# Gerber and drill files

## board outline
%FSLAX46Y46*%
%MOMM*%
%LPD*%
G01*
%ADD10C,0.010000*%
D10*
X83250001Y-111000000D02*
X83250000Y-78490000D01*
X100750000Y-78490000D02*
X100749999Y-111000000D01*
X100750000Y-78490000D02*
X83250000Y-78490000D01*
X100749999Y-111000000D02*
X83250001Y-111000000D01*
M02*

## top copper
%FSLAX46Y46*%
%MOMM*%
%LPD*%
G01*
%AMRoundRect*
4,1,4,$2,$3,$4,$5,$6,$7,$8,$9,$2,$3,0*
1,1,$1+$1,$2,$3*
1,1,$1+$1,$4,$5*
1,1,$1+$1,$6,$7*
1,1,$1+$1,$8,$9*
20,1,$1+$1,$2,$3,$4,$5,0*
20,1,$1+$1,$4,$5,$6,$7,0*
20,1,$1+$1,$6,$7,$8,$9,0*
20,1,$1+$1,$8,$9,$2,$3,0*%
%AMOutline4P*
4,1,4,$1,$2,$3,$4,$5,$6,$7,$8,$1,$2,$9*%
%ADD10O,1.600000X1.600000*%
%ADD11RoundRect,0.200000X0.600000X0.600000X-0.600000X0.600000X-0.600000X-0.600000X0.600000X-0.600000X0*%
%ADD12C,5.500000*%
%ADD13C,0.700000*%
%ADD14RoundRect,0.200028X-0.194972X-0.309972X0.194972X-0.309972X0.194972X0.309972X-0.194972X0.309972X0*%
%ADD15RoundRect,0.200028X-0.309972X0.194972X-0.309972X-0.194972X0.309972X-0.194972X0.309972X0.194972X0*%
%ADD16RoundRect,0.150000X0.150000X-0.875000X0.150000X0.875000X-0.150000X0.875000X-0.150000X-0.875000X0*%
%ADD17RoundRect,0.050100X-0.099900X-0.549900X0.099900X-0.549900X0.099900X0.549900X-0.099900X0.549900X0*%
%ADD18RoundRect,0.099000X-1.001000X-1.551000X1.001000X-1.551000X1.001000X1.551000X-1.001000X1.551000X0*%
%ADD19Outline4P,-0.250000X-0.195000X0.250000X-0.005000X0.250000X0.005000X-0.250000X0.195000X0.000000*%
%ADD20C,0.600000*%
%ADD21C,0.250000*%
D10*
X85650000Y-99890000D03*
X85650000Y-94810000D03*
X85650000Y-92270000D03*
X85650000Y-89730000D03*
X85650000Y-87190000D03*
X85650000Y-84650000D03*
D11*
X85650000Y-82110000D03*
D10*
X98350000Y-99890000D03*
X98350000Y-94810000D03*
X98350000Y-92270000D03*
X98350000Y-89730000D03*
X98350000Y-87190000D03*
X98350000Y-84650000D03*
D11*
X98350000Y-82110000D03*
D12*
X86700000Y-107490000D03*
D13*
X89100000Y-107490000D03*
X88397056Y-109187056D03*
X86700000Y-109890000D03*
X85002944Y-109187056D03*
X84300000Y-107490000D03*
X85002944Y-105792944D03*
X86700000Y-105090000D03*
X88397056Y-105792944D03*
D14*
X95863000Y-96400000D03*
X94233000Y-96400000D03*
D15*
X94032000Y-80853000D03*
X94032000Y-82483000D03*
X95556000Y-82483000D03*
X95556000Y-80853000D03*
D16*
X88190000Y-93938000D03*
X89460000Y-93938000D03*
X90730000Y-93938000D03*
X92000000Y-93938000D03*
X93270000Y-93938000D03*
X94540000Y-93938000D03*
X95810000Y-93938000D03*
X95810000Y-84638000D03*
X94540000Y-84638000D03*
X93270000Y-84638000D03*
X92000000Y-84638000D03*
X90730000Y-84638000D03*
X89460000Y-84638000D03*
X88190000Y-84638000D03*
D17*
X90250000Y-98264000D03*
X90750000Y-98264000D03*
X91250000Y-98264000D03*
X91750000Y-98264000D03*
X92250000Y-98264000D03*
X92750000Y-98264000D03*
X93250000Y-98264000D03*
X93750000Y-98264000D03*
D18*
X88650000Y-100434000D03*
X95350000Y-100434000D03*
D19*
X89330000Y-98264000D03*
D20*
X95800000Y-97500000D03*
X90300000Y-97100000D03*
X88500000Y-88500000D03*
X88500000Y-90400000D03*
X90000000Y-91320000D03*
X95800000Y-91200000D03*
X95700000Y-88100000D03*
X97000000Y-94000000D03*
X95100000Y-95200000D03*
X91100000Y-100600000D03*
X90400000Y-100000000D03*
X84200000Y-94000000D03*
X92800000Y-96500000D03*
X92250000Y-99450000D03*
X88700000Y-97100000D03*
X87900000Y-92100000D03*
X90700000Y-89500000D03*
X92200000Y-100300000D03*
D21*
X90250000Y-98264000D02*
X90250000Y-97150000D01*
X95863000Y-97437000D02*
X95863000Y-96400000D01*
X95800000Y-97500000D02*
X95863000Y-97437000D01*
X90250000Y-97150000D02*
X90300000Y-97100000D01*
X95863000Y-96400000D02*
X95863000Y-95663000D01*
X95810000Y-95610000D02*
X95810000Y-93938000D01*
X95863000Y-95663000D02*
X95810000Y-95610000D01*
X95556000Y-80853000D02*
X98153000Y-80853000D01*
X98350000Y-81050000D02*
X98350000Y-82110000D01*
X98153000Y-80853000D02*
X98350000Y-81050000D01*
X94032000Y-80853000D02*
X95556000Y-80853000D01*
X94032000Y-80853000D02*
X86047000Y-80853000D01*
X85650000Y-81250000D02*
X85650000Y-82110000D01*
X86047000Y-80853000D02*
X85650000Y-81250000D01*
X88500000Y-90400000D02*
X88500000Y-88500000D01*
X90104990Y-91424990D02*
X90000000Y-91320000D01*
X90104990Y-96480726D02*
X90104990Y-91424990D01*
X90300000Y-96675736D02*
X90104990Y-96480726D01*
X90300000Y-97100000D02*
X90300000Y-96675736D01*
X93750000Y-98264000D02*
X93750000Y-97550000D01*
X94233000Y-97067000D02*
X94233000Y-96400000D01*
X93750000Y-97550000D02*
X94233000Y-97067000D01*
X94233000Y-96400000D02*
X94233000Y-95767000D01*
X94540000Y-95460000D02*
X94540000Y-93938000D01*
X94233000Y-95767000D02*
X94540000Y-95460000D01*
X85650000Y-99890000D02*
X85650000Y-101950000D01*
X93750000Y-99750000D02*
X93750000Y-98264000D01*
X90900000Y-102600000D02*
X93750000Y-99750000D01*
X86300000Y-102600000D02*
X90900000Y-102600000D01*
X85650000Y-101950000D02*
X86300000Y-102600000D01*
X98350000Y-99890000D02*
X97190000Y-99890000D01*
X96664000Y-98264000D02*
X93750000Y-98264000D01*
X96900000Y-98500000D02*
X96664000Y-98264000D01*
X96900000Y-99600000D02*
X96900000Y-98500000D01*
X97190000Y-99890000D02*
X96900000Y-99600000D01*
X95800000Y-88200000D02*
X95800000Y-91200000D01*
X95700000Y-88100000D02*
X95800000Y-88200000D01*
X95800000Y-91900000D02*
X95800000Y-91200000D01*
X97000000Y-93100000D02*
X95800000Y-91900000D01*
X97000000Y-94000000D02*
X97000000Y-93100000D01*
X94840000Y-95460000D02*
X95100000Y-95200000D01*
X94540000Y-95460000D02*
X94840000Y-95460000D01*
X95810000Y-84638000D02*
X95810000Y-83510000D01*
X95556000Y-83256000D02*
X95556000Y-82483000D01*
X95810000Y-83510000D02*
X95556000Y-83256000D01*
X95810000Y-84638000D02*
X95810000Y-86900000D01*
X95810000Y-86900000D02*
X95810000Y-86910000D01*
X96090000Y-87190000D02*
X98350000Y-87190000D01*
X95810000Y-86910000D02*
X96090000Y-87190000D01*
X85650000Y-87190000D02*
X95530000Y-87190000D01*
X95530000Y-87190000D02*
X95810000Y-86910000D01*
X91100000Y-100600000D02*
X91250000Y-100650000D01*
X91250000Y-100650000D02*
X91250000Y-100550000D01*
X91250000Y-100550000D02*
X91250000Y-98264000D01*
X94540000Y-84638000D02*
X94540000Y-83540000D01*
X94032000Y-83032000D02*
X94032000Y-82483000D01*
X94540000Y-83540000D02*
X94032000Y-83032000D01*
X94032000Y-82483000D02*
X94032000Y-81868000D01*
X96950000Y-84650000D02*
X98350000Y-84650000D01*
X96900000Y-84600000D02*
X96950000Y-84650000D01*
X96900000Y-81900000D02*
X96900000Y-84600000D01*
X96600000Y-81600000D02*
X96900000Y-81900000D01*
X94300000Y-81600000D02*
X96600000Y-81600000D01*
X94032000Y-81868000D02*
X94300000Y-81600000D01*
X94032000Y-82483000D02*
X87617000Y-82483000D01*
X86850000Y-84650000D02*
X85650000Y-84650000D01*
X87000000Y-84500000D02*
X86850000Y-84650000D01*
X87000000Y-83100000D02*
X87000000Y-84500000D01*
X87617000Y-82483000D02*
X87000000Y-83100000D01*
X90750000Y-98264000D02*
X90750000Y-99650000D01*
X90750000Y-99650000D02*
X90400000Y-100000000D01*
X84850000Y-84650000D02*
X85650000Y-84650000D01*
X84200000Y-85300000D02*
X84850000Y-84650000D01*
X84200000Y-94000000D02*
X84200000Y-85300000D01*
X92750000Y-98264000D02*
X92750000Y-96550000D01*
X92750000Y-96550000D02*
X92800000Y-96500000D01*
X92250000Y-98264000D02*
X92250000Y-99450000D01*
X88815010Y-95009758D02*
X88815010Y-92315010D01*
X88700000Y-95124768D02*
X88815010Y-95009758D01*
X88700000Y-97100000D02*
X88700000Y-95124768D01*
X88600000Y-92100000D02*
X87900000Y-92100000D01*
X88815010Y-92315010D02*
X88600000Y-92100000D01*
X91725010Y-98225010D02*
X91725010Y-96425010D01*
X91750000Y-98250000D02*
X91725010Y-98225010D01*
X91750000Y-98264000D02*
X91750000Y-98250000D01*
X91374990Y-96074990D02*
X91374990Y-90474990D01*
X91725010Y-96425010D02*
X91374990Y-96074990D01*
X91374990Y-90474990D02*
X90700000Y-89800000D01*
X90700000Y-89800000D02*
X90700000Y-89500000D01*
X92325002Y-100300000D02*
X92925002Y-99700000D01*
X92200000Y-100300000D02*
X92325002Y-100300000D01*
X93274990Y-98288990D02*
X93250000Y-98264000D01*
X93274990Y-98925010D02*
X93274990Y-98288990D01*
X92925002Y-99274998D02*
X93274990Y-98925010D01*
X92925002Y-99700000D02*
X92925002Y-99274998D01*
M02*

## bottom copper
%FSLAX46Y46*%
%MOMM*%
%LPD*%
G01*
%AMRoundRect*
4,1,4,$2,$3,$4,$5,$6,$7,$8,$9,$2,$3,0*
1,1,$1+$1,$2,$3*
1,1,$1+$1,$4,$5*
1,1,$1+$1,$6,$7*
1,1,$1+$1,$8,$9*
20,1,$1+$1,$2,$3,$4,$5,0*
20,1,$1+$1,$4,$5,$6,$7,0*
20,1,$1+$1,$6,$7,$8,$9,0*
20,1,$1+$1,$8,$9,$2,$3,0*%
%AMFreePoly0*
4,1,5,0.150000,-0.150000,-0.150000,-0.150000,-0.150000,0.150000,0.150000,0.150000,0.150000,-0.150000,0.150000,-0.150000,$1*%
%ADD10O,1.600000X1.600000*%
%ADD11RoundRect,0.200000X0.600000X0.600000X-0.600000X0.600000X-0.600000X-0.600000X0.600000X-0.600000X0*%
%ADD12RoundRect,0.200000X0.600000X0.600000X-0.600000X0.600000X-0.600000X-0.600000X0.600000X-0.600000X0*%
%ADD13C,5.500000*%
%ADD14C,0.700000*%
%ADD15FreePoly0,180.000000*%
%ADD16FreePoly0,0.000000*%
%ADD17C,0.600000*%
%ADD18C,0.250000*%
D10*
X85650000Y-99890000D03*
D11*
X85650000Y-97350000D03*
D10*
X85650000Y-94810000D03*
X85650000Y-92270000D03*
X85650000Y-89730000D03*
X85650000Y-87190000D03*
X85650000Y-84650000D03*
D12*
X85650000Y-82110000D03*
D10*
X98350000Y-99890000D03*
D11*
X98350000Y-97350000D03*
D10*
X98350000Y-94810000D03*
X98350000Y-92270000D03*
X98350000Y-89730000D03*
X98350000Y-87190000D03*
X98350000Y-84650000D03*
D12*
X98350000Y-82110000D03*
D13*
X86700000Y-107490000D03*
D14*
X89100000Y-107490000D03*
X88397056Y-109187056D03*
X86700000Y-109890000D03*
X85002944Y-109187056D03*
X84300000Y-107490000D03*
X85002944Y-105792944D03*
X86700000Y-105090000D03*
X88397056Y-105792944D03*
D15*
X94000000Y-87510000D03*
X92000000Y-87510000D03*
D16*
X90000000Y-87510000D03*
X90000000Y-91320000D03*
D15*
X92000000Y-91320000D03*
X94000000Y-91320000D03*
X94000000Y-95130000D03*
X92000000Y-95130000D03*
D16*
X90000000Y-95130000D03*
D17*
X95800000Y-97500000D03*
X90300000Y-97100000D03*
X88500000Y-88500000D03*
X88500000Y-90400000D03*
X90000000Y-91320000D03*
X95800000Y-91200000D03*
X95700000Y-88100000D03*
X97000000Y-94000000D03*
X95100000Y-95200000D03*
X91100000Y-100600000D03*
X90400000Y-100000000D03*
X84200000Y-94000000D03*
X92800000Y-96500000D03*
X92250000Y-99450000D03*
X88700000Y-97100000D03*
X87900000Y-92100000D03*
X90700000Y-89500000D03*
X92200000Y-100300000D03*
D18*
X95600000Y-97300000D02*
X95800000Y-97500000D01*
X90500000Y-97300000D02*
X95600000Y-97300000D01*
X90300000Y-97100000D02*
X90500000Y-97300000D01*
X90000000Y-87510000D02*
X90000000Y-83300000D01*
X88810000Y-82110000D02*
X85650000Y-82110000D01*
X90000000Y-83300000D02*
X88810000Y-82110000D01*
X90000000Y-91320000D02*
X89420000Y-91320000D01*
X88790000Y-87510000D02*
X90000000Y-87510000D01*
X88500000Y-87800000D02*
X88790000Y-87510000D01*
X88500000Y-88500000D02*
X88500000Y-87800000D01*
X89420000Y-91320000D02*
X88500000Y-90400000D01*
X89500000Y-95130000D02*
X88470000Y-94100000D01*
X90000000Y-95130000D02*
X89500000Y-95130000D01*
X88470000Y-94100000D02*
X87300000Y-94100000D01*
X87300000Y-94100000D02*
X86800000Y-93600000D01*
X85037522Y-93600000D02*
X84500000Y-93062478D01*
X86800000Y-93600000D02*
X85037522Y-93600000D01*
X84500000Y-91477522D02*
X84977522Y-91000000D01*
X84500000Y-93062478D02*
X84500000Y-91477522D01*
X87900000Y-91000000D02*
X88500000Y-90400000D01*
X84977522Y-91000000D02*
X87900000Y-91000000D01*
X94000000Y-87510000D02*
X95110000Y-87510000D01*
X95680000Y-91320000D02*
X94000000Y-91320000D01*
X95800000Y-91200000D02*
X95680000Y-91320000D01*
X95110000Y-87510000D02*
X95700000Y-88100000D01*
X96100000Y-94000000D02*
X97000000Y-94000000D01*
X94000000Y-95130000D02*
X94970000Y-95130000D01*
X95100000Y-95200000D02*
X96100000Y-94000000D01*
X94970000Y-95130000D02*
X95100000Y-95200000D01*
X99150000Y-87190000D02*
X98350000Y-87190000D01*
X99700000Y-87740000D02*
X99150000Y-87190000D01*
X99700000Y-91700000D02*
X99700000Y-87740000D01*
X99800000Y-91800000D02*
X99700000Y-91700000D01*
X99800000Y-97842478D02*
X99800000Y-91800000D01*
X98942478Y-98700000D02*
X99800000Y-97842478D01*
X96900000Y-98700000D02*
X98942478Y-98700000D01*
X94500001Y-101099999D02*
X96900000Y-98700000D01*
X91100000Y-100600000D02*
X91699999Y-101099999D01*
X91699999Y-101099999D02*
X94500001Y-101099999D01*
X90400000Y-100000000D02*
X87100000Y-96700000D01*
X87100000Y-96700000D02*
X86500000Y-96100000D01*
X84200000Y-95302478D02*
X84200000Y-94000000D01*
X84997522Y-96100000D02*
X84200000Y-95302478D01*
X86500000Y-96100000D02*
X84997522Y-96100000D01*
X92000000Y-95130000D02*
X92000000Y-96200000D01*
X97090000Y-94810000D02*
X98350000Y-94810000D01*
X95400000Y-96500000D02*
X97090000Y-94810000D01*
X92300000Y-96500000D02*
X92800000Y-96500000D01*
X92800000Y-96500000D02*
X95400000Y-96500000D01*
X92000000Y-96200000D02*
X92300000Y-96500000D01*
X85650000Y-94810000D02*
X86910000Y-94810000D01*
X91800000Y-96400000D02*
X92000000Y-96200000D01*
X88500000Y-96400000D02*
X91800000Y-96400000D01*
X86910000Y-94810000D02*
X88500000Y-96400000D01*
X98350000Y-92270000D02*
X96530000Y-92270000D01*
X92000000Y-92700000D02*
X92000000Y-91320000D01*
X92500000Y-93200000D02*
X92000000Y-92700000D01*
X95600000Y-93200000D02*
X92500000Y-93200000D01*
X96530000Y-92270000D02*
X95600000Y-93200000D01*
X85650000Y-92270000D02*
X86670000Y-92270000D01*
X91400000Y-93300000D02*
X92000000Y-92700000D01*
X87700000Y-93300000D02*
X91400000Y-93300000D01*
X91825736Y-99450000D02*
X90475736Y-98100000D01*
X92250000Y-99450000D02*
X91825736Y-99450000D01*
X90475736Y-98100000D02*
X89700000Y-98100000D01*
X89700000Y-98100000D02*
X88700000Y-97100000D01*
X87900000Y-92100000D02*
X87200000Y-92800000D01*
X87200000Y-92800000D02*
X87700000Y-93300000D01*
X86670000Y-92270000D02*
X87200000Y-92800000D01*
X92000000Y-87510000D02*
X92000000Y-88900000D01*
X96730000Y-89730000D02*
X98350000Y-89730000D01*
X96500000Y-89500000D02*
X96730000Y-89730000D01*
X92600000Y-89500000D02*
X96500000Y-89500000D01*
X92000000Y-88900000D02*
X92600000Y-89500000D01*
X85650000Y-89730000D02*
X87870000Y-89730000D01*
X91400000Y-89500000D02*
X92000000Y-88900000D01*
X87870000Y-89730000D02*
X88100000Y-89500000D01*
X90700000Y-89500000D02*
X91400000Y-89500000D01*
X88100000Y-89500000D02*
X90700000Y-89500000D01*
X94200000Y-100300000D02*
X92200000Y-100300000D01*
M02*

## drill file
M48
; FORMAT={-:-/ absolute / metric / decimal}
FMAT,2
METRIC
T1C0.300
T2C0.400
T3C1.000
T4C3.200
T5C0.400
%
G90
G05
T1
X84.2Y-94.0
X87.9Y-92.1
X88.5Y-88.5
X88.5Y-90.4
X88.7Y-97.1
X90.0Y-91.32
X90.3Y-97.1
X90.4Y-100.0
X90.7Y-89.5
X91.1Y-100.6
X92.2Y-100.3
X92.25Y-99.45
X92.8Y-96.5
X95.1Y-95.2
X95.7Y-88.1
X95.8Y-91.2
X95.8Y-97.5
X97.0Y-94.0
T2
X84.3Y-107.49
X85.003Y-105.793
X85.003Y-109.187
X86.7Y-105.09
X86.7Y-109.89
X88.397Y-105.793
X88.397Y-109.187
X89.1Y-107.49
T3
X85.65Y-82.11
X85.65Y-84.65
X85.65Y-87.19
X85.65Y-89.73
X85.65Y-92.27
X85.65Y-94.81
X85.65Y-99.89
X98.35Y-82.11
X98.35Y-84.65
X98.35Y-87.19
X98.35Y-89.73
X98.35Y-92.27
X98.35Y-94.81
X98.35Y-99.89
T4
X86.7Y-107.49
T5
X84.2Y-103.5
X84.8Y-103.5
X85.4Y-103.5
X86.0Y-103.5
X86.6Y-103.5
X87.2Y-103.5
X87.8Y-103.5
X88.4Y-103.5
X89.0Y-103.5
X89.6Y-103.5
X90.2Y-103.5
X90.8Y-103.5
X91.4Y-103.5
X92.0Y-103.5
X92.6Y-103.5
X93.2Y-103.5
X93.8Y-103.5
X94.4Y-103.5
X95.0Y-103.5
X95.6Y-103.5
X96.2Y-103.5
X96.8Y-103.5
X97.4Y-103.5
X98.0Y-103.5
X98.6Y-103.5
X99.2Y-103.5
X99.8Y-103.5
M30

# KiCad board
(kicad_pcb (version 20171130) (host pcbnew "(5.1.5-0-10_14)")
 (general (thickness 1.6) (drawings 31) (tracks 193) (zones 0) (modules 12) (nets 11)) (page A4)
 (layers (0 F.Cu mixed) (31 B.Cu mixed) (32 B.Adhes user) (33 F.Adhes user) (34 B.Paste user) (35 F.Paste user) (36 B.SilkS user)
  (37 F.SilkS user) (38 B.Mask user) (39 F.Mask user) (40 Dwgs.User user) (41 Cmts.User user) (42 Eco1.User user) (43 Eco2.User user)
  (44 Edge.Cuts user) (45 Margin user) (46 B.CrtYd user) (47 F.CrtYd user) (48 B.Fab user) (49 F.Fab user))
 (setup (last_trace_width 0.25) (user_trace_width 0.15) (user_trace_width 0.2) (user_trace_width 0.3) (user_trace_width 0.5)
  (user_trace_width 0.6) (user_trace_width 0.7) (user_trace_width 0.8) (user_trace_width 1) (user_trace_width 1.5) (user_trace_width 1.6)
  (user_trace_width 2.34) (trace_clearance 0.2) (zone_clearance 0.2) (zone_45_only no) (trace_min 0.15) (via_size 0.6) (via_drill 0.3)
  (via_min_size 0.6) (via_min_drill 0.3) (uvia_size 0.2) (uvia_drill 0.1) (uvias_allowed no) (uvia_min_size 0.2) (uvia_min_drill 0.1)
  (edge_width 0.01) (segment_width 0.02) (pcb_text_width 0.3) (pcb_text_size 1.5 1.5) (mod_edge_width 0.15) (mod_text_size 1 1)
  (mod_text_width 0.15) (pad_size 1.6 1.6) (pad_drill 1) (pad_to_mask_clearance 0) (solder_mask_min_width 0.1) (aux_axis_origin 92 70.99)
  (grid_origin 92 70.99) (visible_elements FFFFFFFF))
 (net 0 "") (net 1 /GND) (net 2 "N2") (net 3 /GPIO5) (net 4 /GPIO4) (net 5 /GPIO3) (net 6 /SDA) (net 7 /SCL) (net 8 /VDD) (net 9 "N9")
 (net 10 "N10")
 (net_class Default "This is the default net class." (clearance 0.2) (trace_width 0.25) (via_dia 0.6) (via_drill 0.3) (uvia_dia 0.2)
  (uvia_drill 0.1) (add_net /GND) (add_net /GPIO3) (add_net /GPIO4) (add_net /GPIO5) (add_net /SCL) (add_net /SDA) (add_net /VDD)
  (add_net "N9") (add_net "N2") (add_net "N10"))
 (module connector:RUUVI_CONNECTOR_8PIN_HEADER (layer B.Cu) (at 85.65 82.11 180)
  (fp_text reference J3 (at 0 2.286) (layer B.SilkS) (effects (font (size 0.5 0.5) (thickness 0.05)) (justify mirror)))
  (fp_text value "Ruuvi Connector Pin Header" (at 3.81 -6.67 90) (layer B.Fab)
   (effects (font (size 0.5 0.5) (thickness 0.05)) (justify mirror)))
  (pad 8 thru_hole oval (at 0 -17.78 180) (size 1.6 1.6) (drill 1) (layers *.Cu *.Mask) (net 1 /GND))
  (pad 7 smd roundrect (at 0 -15.24 180) (size 1.6 1.6) (layers B.Cu B.Paste B.Mask) (roundrect_rratio 0.125) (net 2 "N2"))
  (pad 6 thru_hole oval (at 0 -12.7 180) (size 1.6 1.6) (drill 1) (layers *.Cu *.Mask) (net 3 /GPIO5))
  (pad 5 thru_hole oval (at 0 -10.16 180) (size 1.6 1.6) (drill 1) (layers *.Cu *.Mask) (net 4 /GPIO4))
  (pad 4 thru_hole oval (at 0 -7.62 180) (size 1.6 1.6) (drill 1) (layers *.Cu *.Mask) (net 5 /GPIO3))
  (pad 3 thru_hole oval (at 0 -5.08 180) (size 1.6 1.6) (drill 1) (layers *.Cu *.Mask) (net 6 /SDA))
  (pad 2 thru_hole oval (at 0 -2.54 180) (size 1.6 1.6) (drill 1) (layers *.Cu *.Mask) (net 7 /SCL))
  (pad 1 thru_hole roundrect (at 0 0 180) (size 1.6 1.6) (drill 1) (layers *.Cu *.Mask) (roundrect_rratio 0.125) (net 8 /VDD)))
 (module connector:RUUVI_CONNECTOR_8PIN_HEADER (layer B.Cu) (at 98.35 82.11 180)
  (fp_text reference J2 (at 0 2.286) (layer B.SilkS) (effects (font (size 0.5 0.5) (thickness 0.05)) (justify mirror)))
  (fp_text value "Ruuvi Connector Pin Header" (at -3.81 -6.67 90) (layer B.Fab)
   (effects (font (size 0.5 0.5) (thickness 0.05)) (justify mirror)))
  (pad 8 thru_hole oval (at 0 -17.78 180) (size 1.6 1.6) (drill 1) (layers *.Cu *.Mask) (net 1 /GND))
  (pad 7 smd roundrect (at 0 -15.24 180) (size 1.6 1.6) (layers B.Cu B.Paste B.Mask) (roundrect_rratio 0.125) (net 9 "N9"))
  (pad 6 thru_hole oval (at 0 -12.7 180) (size 1.6 1.6) (drill 1) (layers *.Cu *.Mask) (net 3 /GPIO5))
  (pad 5 thru_hole oval (at 0 -10.16 180) (size 1.6 1.6) (drill 1) (layers *.Cu *.Mask) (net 4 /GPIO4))
  (pad 4 thru_hole oval (at 0 -7.62 180) (size 1.6 1.6) (drill 1) (layers *.Cu *.Mask) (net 5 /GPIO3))
  (pad 3 thru_hole oval (at 0 -5.08 180) (size 1.6 1.6) (drill 1) (layers *.Cu *.Mask) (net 6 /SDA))
  (pad 2 thru_hole oval (at 0 -2.54 180) (size 1.6 1.6) (drill 1) (layers *.Cu *.Mask) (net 7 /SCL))
  (pad 1 thru_hole roundrect (at 0 0 180) (size 1.6 1.6) (drill 1) (layers *.Cu *.Mask) (roundrect_rratio 0.125) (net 8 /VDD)))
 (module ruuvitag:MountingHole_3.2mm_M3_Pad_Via (layer F.Cu) (at 86.7 107.49)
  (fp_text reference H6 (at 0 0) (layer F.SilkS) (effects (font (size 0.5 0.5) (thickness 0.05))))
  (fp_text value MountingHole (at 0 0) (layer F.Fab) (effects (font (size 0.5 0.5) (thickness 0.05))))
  (pad 1 thru_hole circle (at 0 0) (size 5.5 5.5) (drill 3.2) (layers *.Cu *.Mask))
  (pad 1 thru_hole circle (at 2.4 0) (size 0.7 0.7) (drill 0.4) (layers *.Cu *.Mask))
  (pad 1 thru_hole circle (at 1.697056 1.697056) (size 0.7 0.7) (drill 0.4) (layers *.Cu *.Mask))
  (pad 1 thru_hole circle (at 0 2.4) (size 0.7 0.7) (drill 0.4) (layers *.Cu *.Mask))
  (pad 1 thru_hole circle (at -1.697056 1.697056) (size 0.7 0.7) (drill 0.4) (layers *.Cu *.Mask))
  (pad 1 thru_hole circle (at -2.4 0) (size 0.7 0.7) (drill 0.4) (layers *.Cu *.Mask))
  (pad 1 thru_hole circle (at -1.697056 -1.697056) (size 0.7 0.7) (drill 0.4) (layers *.Cu *.Mask))
  (pad 1 thru_hole circle (at 0 -2.4) (size 0.7 0.7) (drill 0.4) (layers *.Cu *.Mask))
  (pad 1 thru_hole circle (at 1.697056 -1.697056) (size 0.7 0.7) (drill 0.4) (layers *.Cu *.Mask)))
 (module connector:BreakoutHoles (layer F.Cu) (at 92 103.5)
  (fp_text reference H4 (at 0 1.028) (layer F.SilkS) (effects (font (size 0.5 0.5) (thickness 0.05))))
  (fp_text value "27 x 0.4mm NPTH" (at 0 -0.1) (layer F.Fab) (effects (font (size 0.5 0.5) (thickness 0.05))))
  (pad "" np_thru_hole circle (at -6.6 0) (size 0.4 0.4) (drill 0.4) (layers *.Cu *.Mask))
  (pad "" np_thru_hole circle (at -0.6 0) (size 0.4 0.4) (drill 0.4) (layers *.Cu *.Mask))
  (pad "" np_thru_hole circle (at -3.6 0) (size 0.4 0.4) (drill 0.4) (layers *.Cu *.Mask))
  (pad "" np_thru_hole circle (at -1.2 0) (size 0.4 0.4) (drill 0.4) (layers *.Cu *.Mask))
  (pad "" np_thru_hole circle (at -3 0) (size 0.4 0.4) (drill 0.4) (layers *.Cu *.Mask))
  (pad "" np_thru_hole circle (at -1.8 0) (size 0.4 0.4) (drill 0.4) (layers *.Cu *.Mask))
  (pad "" np_thru_hole circle (at -4.8 0) (size 0.4 0.4) (drill 0.4) (layers *.Cu *.Mask))
  (pad "" np_thru_hole circle (at -5.4 0) (size 0.4 0.4) (drill 0.4) (layers *.Cu *.Mask))
  (pad "" np_thru_hole circle (at -7.8 0) (size 0.4 0.4) (drill 0.4) (layers *.Cu *.Mask))
  (pad "" np_thru_hole circle (at -2.4 0) (size 0.4 0.4) (drill 0.4) (layers *.Cu *.Mask))
  (pad "" np_thru_hole circle (at -4.2 0) (size 0.4 0.4) (drill 0.4) (layers *.Cu *.Mask))
  (pad "" np_thru_hole circle (at -7.2 0) (size 0.4 0.4) (drill 0.4) (layers *.Cu *.Mask))
  (pad "" np_thru_hole circle (at -6 0) (size 0.4 0.4) (drill 0.4) (layers *.Cu *.Mask))
  (pad "" np_thru_hole circle (at 7.8 0) (size 0.4 0.4) (drill 0.4) (layers *.Cu *.Mask))
  (pad "" np_thru_hole circle (at 7.2 0) (size 0.4 0.4) (drill 0.4) (layers *.Cu *.Mask))
  (pad "" np_thru_hole circle (at 6.6 0) (size 0.4 0.4) (drill 0.4) (layers *.Cu *.Mask))
  (pad "" np_thru_hole circle (at 6 0) (size 0.4 0.4) (drill 0.4) (layers *.Cu *.Mask))
  (pad "" np_thru_hole circle (at 5.4 0) (size 0.4 0.4) (drill 0.4) (layers *.Cu *.Mask))
  (pad "" np_thru_hole circle (at 4.8 0) (size 0.4 0.4) (drill 0.4) (layers *.Cu *.Mask))
  (pad "" np_thru_hole circle (at 4.2 0) (size 0.4 0.4) (drill 0.4) (layers *.Cu *.Mask))
  (pad "" np_thru_hole circle (at 3.6 0) (size 0.4 0.4) (drill 0.4) (layers *.Cu *.Mask))
  (pad "" np_thru_hole circle (at 3 0) (size 0.4 0.4) (drill 0.4) (layers *.Cu *.Mask))
  (pad "" np_thru_hole circle (at 2.4 0) (size 0.4 0.4) (drill 0.4) (layers *.Cu *.Mask))
  (pad "" np_thru_hole circle (at 1.8 0) (size 0.4 0.4) (drill 0.4) (layers *.Cu *.Mask))
  (pad "" np_thru_hole circle (at 1.2 0) (size 0.4 0.4) (drill 0.4) (layers *.Cu *.Mask))
  (pad "" np_thru_hole circle (at 0.6 0) (size 0.4 0.4) (drill 0.4) (layers *.Cu *.Mask))
  (pad "" np_thru_hole circle (at 0 0) (size 0.4 0.4) (drill 0.4) (layers *.Cu *.Mask)))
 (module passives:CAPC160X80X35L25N (layer F.Cu) (at 95.048 96.4)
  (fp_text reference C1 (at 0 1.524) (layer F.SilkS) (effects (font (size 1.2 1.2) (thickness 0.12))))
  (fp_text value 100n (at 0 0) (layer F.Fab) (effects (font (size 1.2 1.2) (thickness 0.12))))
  (pad 2 smd roundrect (at 0.815 0) (size 0.79 1.02) (layers F.Cu F.Paste F.Mask) (roundrect_rratio 0.2532) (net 8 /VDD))
  (pad 1 smd roundrect (at -0.815 0) (size 0.79 1.02) (layers F.Cu F.Paste F.Mask) (roundrect_rratio 0.2532) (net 1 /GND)))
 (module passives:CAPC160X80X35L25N (layer F.Cu) (at 94.032 81.668 270)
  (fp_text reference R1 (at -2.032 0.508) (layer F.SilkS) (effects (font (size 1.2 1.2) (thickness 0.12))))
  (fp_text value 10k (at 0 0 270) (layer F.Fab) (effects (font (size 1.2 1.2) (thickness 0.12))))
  (pad 1 smd roundrect (at -0.815 0 270) (size 0.79 1.02) (layers F.Cu F.Paste F.Mask) (roundrect_rratio 0.2532) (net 8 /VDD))
  (pad 2 smd roundrect (at 0.815 0 270) (size 0.79 1.02) (layers F.Cu F.Paste F.Mask) (roundrect_rratio 0.2532) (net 7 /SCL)))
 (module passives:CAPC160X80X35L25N (layer F.Cu) (at 95.556 81.668 270)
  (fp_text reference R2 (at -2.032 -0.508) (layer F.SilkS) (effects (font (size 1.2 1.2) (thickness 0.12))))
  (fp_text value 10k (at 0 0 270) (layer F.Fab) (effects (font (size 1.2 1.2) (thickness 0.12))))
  (pad 2 smd roundrect (at 0.815 0 270) (size 0.79 1.02) (layers F.Cu F.Paste F.Mask) (roundrect_rratio 0.2532) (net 6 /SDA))
  (pad 1 smd roundrect (at -0.815 0 270) (size 0.79 1.02) (layers F.Cu F.Paste F.Mask) (roundrect_rratio 0.2532) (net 8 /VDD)))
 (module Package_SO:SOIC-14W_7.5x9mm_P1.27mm (layer F.Cu) (at 92 89.288 90)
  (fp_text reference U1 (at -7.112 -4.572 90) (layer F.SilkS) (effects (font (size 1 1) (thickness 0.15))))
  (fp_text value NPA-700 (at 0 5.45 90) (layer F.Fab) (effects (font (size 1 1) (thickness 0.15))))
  (pad 1 smd roundrect (at -4.65 -3.81 90) (size 2.05 0.6) (layers F.Cu F.Paste F.Mask) (roundrect_rratio 0.25))
  (pad 2 smd roundrect (at -4.65 -2.54 90) (size 2.05 0.6) (layers F.Cu F.Paste F.Mask) (roundrect_rratio 0.25))
  (pad 3 smd roundrect (at -4.65 -1.27 90) (size 2.05 0.6) (layers F.Cu F.Paste F.Mask) (roundrect_rratio 0.25))
  (pad 4 smd roundrect (at -4.65 0 90) (size 2.05 0.6) (layers F.Cu F.Paste F.Mask) (roundrect_rratio 0.25))
  (pad 5 smd roundrect (at -4.65 1.27 90) (size 2.05 0.6) (layers F.Cu F.Paste F.Mask) (roundrect_rratio 0.25))
  (pad 6 smd roundrect (at -4.65 2.54 90) (size 2.05 0.6) (layers F.Cu F.Paste F.Mask) (roundrect_rratio 0.25) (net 1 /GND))
  (pad 7 smd roundrect (at -4.65 3.81 90) (size 2.05 0.6) (layers F.Cu F.Paste F.Mask) (roundrect_rratio 0.25) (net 8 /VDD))
  (pad 8 smd roundrect (at 4.65 3.81 90) (size 2.05 0.6) (layers F.Cu F.Paste F.Mask) (roundrect_rratio 0.25) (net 6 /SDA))
  (pad 9 smd roundrect (at 4.65 2.54 90) (size 2.05 0.6) (layers F.Cu F.Paste F.Mask) (roundrect_rratio 0.25) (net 7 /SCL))
  (pad 10 smd roundrect (at 4.65 1.27 90) (size 2.05 0.6) (layers F.Cu F.Paste F.Mask) (roundrect_rratio 0.25))
  (pad 11 smd roundrect (at 4.65 0 90) (size 2.05 0.6) (layers F.Cu F.Paste F.Mask) (roundrect_rratio 0.25))
  (pad 12 smd roundrect (at 4.65 -1.27 90) (size 2.05 0.6) (layers F.Cu F.Paste F.Mask) (roundrect_rratio 0.25))
  (pad 13 smd roundrect (at 4.65 -2.54 90) (size 2.05 0.6) (layers F.Cu F.Paste F.Mask) (roundrect_rratio 0.25))
  (pad 14 smd roundrect (at 4.65 -3.81 90) (size 2.05 0.6) (layers F.Cu F.Paste F.Mask) (roundrect_rratio 0.25)))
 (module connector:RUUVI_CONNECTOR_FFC (layer F.Cu) (at 92 100.464)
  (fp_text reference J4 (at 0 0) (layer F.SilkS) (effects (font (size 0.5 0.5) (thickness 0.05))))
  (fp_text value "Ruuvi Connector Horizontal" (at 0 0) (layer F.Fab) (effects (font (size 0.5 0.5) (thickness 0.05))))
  (pad 1 smd roundrect (at -1.75 -2.2) (size 0.3 1.2) (layers F.Cu F.Paste F.Mask) (roundrect_rratio 0.167) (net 8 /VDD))
  (pad 2 smd roundrect (at -1.25 -2.2) (size 0.3 1.2) (layers F.Cu F.Paste F.Mask) (roundrect_rratio 0.167) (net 7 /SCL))
  (pad 3 smd roundrect (at -0.75 -2.2) (size 0.3 1.2) (layers F.Cu F.Paste F.Mask) (roundrect_rratio 0.167) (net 6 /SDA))
  (pad 4 smd roundrect (at -0.25 -2.2) (size 0.3 1.2) (layers F.Cu F.Paste F.Mask) (roundrect_rratio 0.167) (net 5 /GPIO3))
  (pad 5 smd roundrect (at 0.25 -2.2) (size 0.3 1.2) (layers F.Cu F.Paste F.Mask) (roundrect_rratio 0.167) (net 4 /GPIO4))
  (pad 6 smd roundrect (at 0.75 -2.2) (size 0.3 1.2) (layers F.Cu F.Paste F.Mask) (roundrect_rratio 0.167) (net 3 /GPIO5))
  (pad 7 smd roundrect (at 1.25 -2.2) (size 0.3 1.2) (layers F.Cu F.Paste F.Mask) (roundrect_rratio 0.167) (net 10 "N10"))
  (pad 8 smd roundrect (at 1.75 -2.2) (size 0.3 1.2) (layers F.Cu F.Paste F.Mask) (roundrect_rratio 0.167) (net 1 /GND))
  (pad ~ smd roundrect (at -3.35 -0.03) (size 2.2 3.3) (layers F.Cu F.Paste F.Mask) (roundrect_rratio 0.045))
  (pad ~ smd roundrect (at 3.35 -0.03) (size 2.2 3.3) (layers F.Cu F.Paste F.Mask) (roundrect_rratio 0.045))
  (pad ~ smd trapezoid (at -2.67 -2.2) (size 0.5 0.2) (rect_delta 0.19 0) (layers F.Cu F.Mask)))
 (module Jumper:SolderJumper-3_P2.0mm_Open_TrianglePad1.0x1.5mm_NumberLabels (layer B.Cu) (at 92 87.51 180)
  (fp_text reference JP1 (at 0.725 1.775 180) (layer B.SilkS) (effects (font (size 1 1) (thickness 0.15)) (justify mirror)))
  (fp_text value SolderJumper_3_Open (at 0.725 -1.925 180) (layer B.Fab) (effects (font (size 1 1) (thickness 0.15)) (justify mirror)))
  (pad "" smd rect (at 1.2 0 180) (size 1.5 1.5) (layers B.Mask))
  (pad "" smd rect (at -1.2 0 180) (size 1.5 1.5) (layers B.Mask))
  (pad 1 smd custom (at -2 0 180) (size 0.3 0.3) (layers B.Cu B.Mask) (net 1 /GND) (zone_connect 2)
   (options (clearance outline) (anchor rect)) (primitives))
  (pad 2 smd custom (at 0 0 180) (size 0.3 0.3) (layers B.Cu) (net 5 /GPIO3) (zone_connect 2) (options (clearance outline) (anchor rect))
   (primitives))
  (pad 3 smd custom (at 2 0) (size 0.3 0.3) (layers B.Cu B.Mask) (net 8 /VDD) (zone_connect 2) (options (clearance outline) (anchor rect))
   (primitives)))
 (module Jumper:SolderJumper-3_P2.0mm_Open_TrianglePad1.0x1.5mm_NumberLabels (layer B.Cu) (at 92 91.32 180)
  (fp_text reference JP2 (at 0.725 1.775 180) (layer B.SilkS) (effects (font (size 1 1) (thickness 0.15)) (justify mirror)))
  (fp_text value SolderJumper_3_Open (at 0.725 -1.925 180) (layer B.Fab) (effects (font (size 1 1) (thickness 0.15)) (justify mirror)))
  (pad 3 smd custom (at 2 0) (size 0.3 0.3) (layers B.Cu B.Mask) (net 8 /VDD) (zone_connect 2) (options (clearance outline) (anchor rect))
   (primitives))
  (pad 2 smd custom (at 0 0 180) (size 0.3 0.3) (layers B.Cu) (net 4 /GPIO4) (zone_connect 2) (options (clearance outline) (anchor rect))
   (primitives))
  (pad 1 smd custom (at -2 0 180) (size 0.3 0.3) (layers B.Cu B.Mask) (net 1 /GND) (zone_connect 2)
   (options (clearance outline) (anchor rect)) (primitives))
  (pad "" smd rect (at -1.2 0 180) (size 1.5 1.5) (layers B.Mask))
  (pad "" smd rect (at 1.2 0 180) (size 1.5 1.5) (layers B.Mask)))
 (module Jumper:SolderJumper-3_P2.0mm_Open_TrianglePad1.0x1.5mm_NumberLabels (layer B.Cu) (at 92 95.13 180)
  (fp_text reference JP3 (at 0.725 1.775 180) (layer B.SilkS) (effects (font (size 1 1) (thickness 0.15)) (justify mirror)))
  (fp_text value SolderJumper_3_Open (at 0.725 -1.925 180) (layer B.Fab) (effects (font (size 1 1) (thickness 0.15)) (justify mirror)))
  (pad "" smd rect (at 1.2 0 180) (size 1.5 1.5) (layers B.Mask))
  (pad "" smd rect (at -1.2 0 180) (size 1.5 1.5) (layers B.Mask))
  (pad 1 smd custom (at -2 0 180) (size 0.3 0.3) (layers B.Cu B.Mask) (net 1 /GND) (zone_connect 2)
   (options (clearance outline) (anchor rect)) (primitives))
  (pad 2 smd custom (at 0 0 180) (size 0.3 0.3) (layers B.Cu) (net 3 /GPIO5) (zone_connect 2) (options (clearance outline) (anchor rect))
   (primitives))
  (pad 3 smd custom (at 2 0) (size 0.3 0.3) (layers B.Cu B.Mask) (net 8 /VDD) (zone_connect 2) (options (clearance outline) (anchor rect))
   (primitives)))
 (gr_line (start 83.250001 111) (end 83.25 78.49) (layer Edge.Cuts) (width 0.01))
 (gr_line (start 100.75 78.49) (end 100.749999 111) (layer Edge.Cuts) (width 0.01))
 (gr_line (start 100.75 78.49) (end 83.25 78.49) (layer Edge.Cuts) (width 0.01))
 (gr_line (start 100.749999 111) (end 83.250001 111) (layer Edge.Cuts) (width 0.01))
 (segment (start 90.25 98.264) (end 90.25 97.15) (width 0.25) (layer F.Cu) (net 8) (status 400000))
 (segment (start 95.863 97.437) (end 95.863 96.4) (width 0.25) (layer F.Cu) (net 8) (status 800000))
 (segment (start 95.8 97.5) (end 95.863 97.437) (width 0.25) (layer F.Cu) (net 8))
 (via (at 95.8 97.5) (size 0.6) (drill 0.3) (layers F.Cu B.Cu) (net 8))
 (segment (start 95.6 97.3) (end 95.8 97.5) (width 0.25) (layer B.Cu) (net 8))
 (segment (start 90.5 97.3) (end 95.6 97.3) (width 0.25) (layer B.Cu) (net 8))
 (segment (start 90.3 97.1) (end 90.5 97.3) (width 0.25) (layer B.Cu) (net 8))
 (via (at 90.3 97.1) (size 0.6) (drill 0.3) (layers F.Cu B.Cu) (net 8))
 (segment (start 90.25 97.15) (end 90.3 97.1) (width 0.25) (layer F.Cu) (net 8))
 (segment (start 95.863 96.4) (end 95.863 95.663) (width 0.25) (layer F.Cu) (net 8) (status 400000))
 (segment (start 95.81 95.61) (end 95.81 93.938) (width 0.25) (layer F.Cu) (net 8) (status 800000))
 (segment (start 95.863 95.663) (end 95.81 95.61) (width 0.25) (layer F.Cu) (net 8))
 (segment (start 95.556 80.853) (end 98.153 80.853) (width 0.25) (layer F.Cu) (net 8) (status 400000))
 (segment (start 98.35 81.05) (end 98.35 82.11) (width 0.25) (layer F.Cu) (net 8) (status 800000))
 (segment (start 98.153 80.853) (end 98.35 81.05) (width 0.25) (layer F.Cu) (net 8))
 (segment (start 94.032 80.853) (end 95.556 80.853) (width 0.25) (layer F.Cu) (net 8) (status C00000))
 (segment (start 94.032 80.853) (end 86.047 80.853) (width 0.25) (layer F.Cu) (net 8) (status 400000))
 (segment (start 85.65 81.25) (end 85.65 82.11) (width 0.25) (layer F.Cu) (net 8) (status 800000))
 (segment (start 86.047 80.853) (end 85.65 81.25) (width 0.25) (layer F.Cu) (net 8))
 (segment (start 90 87.51) (end 90 83.3) (width 0.25) (layer B.Cu) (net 8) (status 400000))
 (segment (start 88.81 82.11) (end 85.65 82.11) (width 0.25) (layer B.Cu) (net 8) (status 800000))
 (segment (start 90 83.3) (end 88.81 82.11) (width 0.25) (layer B.Cu) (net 8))
 (segment (start 90 91.32) (end 89.42 91.32) (width 0.25) (layer B.Cu) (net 8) (status 400000))
 (segment (start 88.79 87.51) (end 90 87.51) (width 0.25) (layer B.Cu) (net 8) (status 800000))
 (segment (start 88.5 87.8) (end 88.79 87.51) (width 0.25) (layer B.Cu) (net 8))
 (segment (start 88.5 88.5) (end 88.5 87.8) (width 0.25) (layer B.Cu) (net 8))
 (via (at 88.5 88.5) (size 0.6) (drill 0.3) (layers F.Cu B.Cu) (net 8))
 (segment (start 88.5 90.4) (end 88.5 88.5) (width 0.25) (layer F.Cu) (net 8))
 (via (at 88.5 90.4) (size 0.6) (drill 0.3) (layers F.Cu B.Cu) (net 8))
 (segment (start 89.42 91.32) (end 88.5 90.4) (width 0.25) (layer B.Cu) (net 8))
 (via (at 90 91.32) (size 0.6) (drill 0.3) (layers F.Cu B.Cu) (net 8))
 (segment (start 90.10499 91.42499) (end 90 91.32) (width 0.25) (layer F.Cu) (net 8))
 (segment (start 90.10499 96.480726) (end 90.10499 91.42499) (width 0.25) (layer F.Cu) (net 8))
 (segment (start 90.3 96.675736) (end 90.10499 96.480726) (width 0.25) (layer F.Cu) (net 8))
 (segment (start 90.3 97.1) (end 90.3 96.675736) (width 0.25) (layer F.Cu) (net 8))
 (segment (start 89.5 95.13) (end 88.47 94.1) (width 0.25) (layer B.Cu) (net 8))
 (segment (start 90 95.13) (end 89.5 95.13) (width 0.25) (layer B.Cu) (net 8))
 (segment (start 88.47 94.1) (end 87.3 94.1) (width 0.25) (layer B.Cu) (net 8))
 (segment (start 87.3 94.1) (end 86.8 93.6) (width 0.25) (layer B.Cu) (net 8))
 (segment (start 85.037522 93.6) (end 84.5 93.062478) (width 0.25) (layer B.Cu) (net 8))
 (segment (start 86.8 93.6) (end 85.037522 93.6) (width 0.25) (layer B.Cu) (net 8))
 (segment (start 84.5 91.477522) (end 84.977522 91) (width 0.25) (layer B.Cu) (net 8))
 (segment (start 84.5 93.062478) (end 84.5 91.477522) (width 0.25) (layer B.Cu) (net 8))
 (segment (start 87.9 91) (end 88.5 90.4) (width 0.25) (layer B.Cu) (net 8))
 (segment (start 84.977522 91) (end 87.9 91) (width 0.25) (layer B.Cu) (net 8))
 (segment (start 93.75 98.264) (end 93.75 97.55) (width 0.25) (layer F.Cu) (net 1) (status 400000))
 (segment (start 94.233 97.067) (end 94.233 96.4) (width 0.25) (layer F.Cu) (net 1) (status 800000))
 (segment (start 93.75 97.55) (end 94.233 97.067) (width 0.25) (layer F.Cu) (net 1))
 (segment (start 94.233 96.4) (end 94.233 95.767) (width 0.25) (layer F.Cu) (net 1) (status 400000))
 (segment (start 94.54 95.46) (end 94.54 93.938) (width 0.25) (layer F.Cu) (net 1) (status 800000))
 (segment (start 94.233 95.767) (end 94.54 95.46) (width 0.25) (layer F.Cu) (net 1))
 (segment (start 85.65 99.89) (end 85.65 101.95) (width 0.25) (layer F.Cu) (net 1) (status 400000))
 (segment (start 93.75 99.75) (end 93.75 98.264) (width 0.25) (layer F.Cu) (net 1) (status 800000))
 (segment (start 90.9 102.6) (end 93.75 99.75) (width 0.25) (layer F.Cu) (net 1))
 (segment (start 86.3 102.6) (end 90.9 102.6) (width 0.25) (layer F.Cu) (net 1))
 (segment (start 85.65 101.95) (end 86.3 102.6) (width 0.25) (layer F.Cu) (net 1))
 (segment (start 98.35 99.89) (end 97.19 99.89) (width 0.25) (layer F.Cu) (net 1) (status 400000))
 (segment (start 96.664 98.264) (end 93.75 98.264) (width 0.25) (layer F.Cu) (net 1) (status 800000))
 (segment (start 96.9 98.5) (end 96.664 98.264) (width 0.25) (layer F.Cu) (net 1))
 (segment (start 96.9 99.6) (end 96.9 98.5) (width 0.25) (layer F.Cu) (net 1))
 (segment (start 97.19 99.89) (end 96.9 99.6) (width 0.25) (layer F.Cu) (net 1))
 (segment (start 94 87.51) (end 95.11 87.51) (width 0.25) (layer B.Cu) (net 1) (status 400000))
 (segment (start 95.68 91.32) (end 94 91.32) (width 0.25) (layer B.Cu) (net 1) (status 800000))
 (segment (start 95.8 91.2) (end 95.68 91.32) (width 0.25) (layer B.Cu) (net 1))
 (via (at 95.8 91.2) (size 0.6) (drill 0.3) (layers F.Cu B.Cu) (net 1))
 (segment (start 95.8 88.2) (end 95.8 91.2) (width 0.25) (layer F.Cu) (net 1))
 (segment (start 95.7 88.1) (end 95.8 88.2) (width 0.25) (layer F.Cu) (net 1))
 (via (at 95.7 88.1) (size 0.6) (drill 0.3) (layers F.Cu B.Cu) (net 1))
 (segment (start 95.11 87.51) (end 95.7 88.1) (width 0.25) (layer B.Cu) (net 1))
 (segment (start 95.8 91.9) (end 95.8 91.2) (width 0.25) (layer F.Cu) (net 1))
 (segment (start 97 93.1) (end 95.8 91.9) (width 0.25) (layer F.Cu) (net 1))
 (segment (start 97 94) (end 97 93.1) (width 0.25) (layer F.Cu) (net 1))
 (via (at 97 94) (size 0.6) (drill 0.3) (layers F.Cu B.Cu) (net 1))
 (segment (start 96.1 94) (end 97 94) (width 0.25) (layer B.Cu) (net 1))
 (segment (start 94 95.13) (end 94.97 95.13) (width 0.25) (layer B.Cu) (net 1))
 (via (at 95.1 95.2) (size 0.6) (drill 0.3) (layers F.Cu B.Cu) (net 1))
 (segment (start 94.84 95.46) (end 95.1 95.2) (width 0.25) (layer F.Cu) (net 1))
 (segment (start 94.54 95.46) (end 94.84 95.46) (width 0.25) (layer F.Cu) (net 1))
 (segment (start 95.1 95.2) (end 96.1 94) (width 0.25) (layer B.Cu) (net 1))
 (segment (start 94.97 95.13) (end 95.1 95.2) (width 0.25) (layer B.Cu) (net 1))
 (segment (start 95.81 84.638) (end 95.81 83.51) (width 0.25) (layer F.Cu) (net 6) (status 400000))
 (segment (start 95.556 83.256) (end 95.556 82.483) (width 0.25) (layer F.Cu) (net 6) (status 800000))
 (segment (start 95.81 83.51) (end 95.556 83.256) (width 0.25) (layer F.Cu) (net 6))
 (segment (start 95.81 84.638) (end 95.81 86.9) (width 0.25) (layer F.Cu) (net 6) (status 400000))
 (segment (start 95.81 86.9) (end 95.81 86.91) (width 0.25) (layer F.Cu) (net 6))
 (segment (start 96.09 87.19) (end 98.35 87.19) (width 0.25) (layer F.Cu) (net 6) (status 800000))
 (segment (start 95.81 86.91) (end 96.09 87.19) (width 0.25) (layer F.Cu) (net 6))
 (segment (start 85.65 87.19) (end 95.53 87.19) (width 0.25) (layer F.Cu) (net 6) (status 400000))
 (segment (start 95.53 87.19) (end 95.81 86.91) (width 0.25) (layer F.Cu) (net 6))
 (segment (start 99.15 87.19) (end 98.35 87.19) (width 0.25) (layer B.Cu) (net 6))
 (segment (start 99.7 87.74) (end 99.15 87.19) (width 0.25) (layer B.Cu) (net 6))
 (segment (start 99.7 91.7) (end 99.7 87.74) (width 0.25) (layer B.Cu) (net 6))
 (segment (start 99.8 91.8) (end 99.7 91.7) (width 0.25) (layer B.Cu) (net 6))
 (segment (start 99.8 97.842478) (end 99.8 91.8) (width 0.25) (layer B.Cu) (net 6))
 (segment (start 91.1 100.6) (end 91.25 100.65) (width 0.25) (layer F.Cu) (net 6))
 (segment (start 98.942478 98.7) (end 99.8 97.842478) (width 0.25) (layer B.Cu) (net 6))
 (segment (start 96.9 98.7) (end 98.942478 98.7) (width 0.25) (layer B.Cu) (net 6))
 (segment (start 94.500001 101.099999) (end 96.9 98.7) (width 0.25) (layer B.Cu) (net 6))
 (segment (start 91.1 100.6) (end 91.699999 101.099999) (width 0.25) (layer B.Cu) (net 6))
 (segment (start 91.699999 101.099999) (end 94.500001 101.099999) (width 0.25) (layer B.Cu) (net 6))
 (segment (start 91.25 100.65) (end 91.25 100.55) (width 0.25) (layer F.Cu) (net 6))
 (segment (start 91.25 100.55) (end 91.25 98.264) (width 0.25) (layer F.Cu) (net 6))
 (via (at 91.1 100.6) (size 0.6) (drill 0.3) (layers F.Cu B.Cu) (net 6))
 (segment (start 94.54 84.638) (end 94.54 83.54) (width 0.25) (layer F.Cu) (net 7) (status 400000))
 (segment (start 94.032 83.032) (end 94.032 82.483) (width 0.25) (layer F.Cu) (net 7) (status 800000))
 (segment (start 94.54 83.54) (end 94.032 83.032) (width 0.25) (layer F.Cu) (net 7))
 (segment (start 94.032 82.483) (end 94.032 81.868) (width 0.25) (layer F.Cu) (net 7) (status 400000))
 (segment (start 96.95 84.65) (end 98.35 84.65) (width 0.25) (layer F.Cu) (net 7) (status 800000))
 (segment (start 96.9 84.6) (end 96.95 84.65) (width 0.25) (layer F.Cu) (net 7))
 (segment (start 96.9 81.9) (end 96.9 84.6) (width 0.25) (layer F.Cu) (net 7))
 (segment (start 96.6 81.6) (end 96.9 81.9) (width 0.25) (layer F.Cu) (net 7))
 (segment (start 94.3 81.6) (end 96.6 81.6) (width 0.25) (layer F.Cu) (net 7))
 (segment (start 94.032 81.868) (end 94.3 81.6) (width 0.25) (layer F.Cu) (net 7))
 (segment (start 94.032 82.483) (end 87.617 82.483) (width 0.25) (layer F.Cu) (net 7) (status 400000))
 (segment (start 86.85 84.65) (end 85.65 84.65) (width 0.25) (layer F.Cu) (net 7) (status 800000))
 (segment (start 87 84.5) (end 86.85 84.65) (width 0.25) (layer F.Cu) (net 7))
 (segment (start 87 83.1) (end 87 84.5) (width 0.25) (layer F.Cu) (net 7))
 (segment (start 87.617 82.483) (end 87 83.1) (width 0.25) (layer F.Cu) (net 7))
 (segment (start 90.75 98.264) (end 90.75 99.65) (width 0.25) (layer F.Cu) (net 7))
 (via (at 90.4 100) (size 0.6) (drill 0.3) (layers F.Cu B.Cu) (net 7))
 (segment (start 90.75 99.65) (end 90.4 100) (width 0.25) (layer F.Cu) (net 7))
 (segment (start 90.4 100) (end 87.1 96.7) (width 0.25) (layer B.Cu) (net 7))
 (segment (start 87.1 96.7) (end 86.5 96.1) (width 0.25) (layer B.Cu) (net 7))
 (via (at 84.2 94) (size 0.6) (drill 0.3) (layers F.Cu B.Cu) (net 7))
 (segment (start 84.2 95.302478) (end 84.2 94) (width 0.25) (layer B.Cu) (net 7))
 (segment (start 84.997522 96.1) (end 84.2 95.302478) (width 0.25) (layer B.Cu) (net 7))
 (segment (start 86.5 96.1) (end 84.997522 96.1) (width 0.25) (layer B.Cu) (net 7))
 (segment (start 84.85 84.65) (end 85.65 84.65) (width 0.25) (layer F.Cu) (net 7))
 (segment (start 84.2 85.3) (end 84.85 84.65) (width 0.25) (layer F.Cu) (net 7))
 (segment (start 84.2 94) (end 84.2 85.3) (width 0.25) (layer F.Cu) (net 7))
 (segment (start 92 95.13) (end 92 96.2) (width 0.25) (layer B.Cu) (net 3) (status 400000))
 (segment (start 97.09 94.81) (end 98.35 94.81) (width 0.25) (layer B.Cu) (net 3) (status 800000))
 (segment (start 95.4 96.5) (end 97.09 94.81) (width 0.25) (layer B.Cu) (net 3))
 (segment (start 92.3 96.5) (end 92.8 96.5) (width 0.25) (layer B.Cu) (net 3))
 (segment (start 92.8 96.5) (end 95.4 96.5) (width 0.25) (layer B.Cu) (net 3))
 (segment (start 92 96.2) (end 92.3 96.5) (width 0.25) (layer B.Cu) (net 3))
 (segment (start 85.65 94.81) (end 86.91 94.81) (width 0.25) (layer B.Cu) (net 3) (status 400000))
 (segment (start 91.8 96.4) (end 92 96.2) (width 0.25) (layer B.Cu) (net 3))
 (segment (start 88.5 96.4) (end 91.8 96.4) (width 0.25) (layer B.Cu) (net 3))
 (segment (start 86.91 94.81) (end 88.5 96.4) (width 0.25) (layer B.Cu) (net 3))
 (segment (start 92.75 98.264) (end 92.75 96.55) (width 0.25) (layer F.Cu) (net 3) (status 400000))
 (via (at 92.8 96.5) (size 0.6) (drill 0.3) (layers F.Cu B.Cu) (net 3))
 (segment (start 92.75 96.55) (end 92.8 96.5) (width 0.25) (layer F.Cu) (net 3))
 (segment (start 98.35 92.27) (end 96.53 92.27) (width 0.25) (layer B.Cu) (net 4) (status 400000))
 (segment (start 92 92.7) (end 92 91.32) (width 0.25) (layer B.Cu) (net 4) (status 800000))
 (segment (start 92.5 93.2) (end 92 92.7) (width 0.25) (layer B.Cu) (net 4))
 (segment (start 95.6 93.2) (end 92.5 93.2) (width 0.25) (layer B.Cu) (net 4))
 (segment (start 96.53 92.27) (end 95.6 93.2) (width 0.25) (layer B.Cu) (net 4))
 (segment (start 85.65 92.27) (end 86.67 92.27) (width 0.25) (layer B.Cu) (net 4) (status 400000))
 (segment (start 91.4 93.3) (end 92 92.7) (width 0.25) (layer B.Cu) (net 4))
 (segment (start 87.7 93.3) (end 91.4 93.3) (width 0.25) (layer B.Cu) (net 4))
 (segment (start 92.25 98.264) (end 92.25 99.45) (width 0.25) (layer F.Cu) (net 4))
 (via (at 92.25 99.45) (size 0.6) (drill 0.3) (layers F.Cu B.Cu) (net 4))
 (segment (start 91.825736 99.45) (end 90.475736 98.1) (width 0.25) (layer B.Cu) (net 4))
 (segment (start 92.25 99.45) (end 91.825736 99.45) (width 0.25) (layer B.Cu) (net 4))
 (segment (start 90.475736 98.1) (end 89.7 98.1) (width 0.25) (layer B.Cu) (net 4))
 (via (at 88.7 97.1) (size 0.6) (drill 0.3) (layers F.Cu B.Cu) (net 4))
 (segment (start 89.7 98.1) (end 88.7 97.1) (width 0.25) (layer B.Cu) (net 4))
 (segment (start 88.81501 95.009758) (end 88.81501 92.31501) (width 0.25) (layer F.Cu) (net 4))
 (segment (start 88.7 95.124768) (end 88.81501 95.009758) (width 0.25) (layer F.Cu) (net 4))
 (segment (start 88.7 97.1) (end 88.7 95.124768) (width 0.25) (layer F.Cu) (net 4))
 (via (at 87.9 92.1) (size 0.6) (drill 0.3) (layers F.Cu B.Cu) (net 4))
 (segment (start 88.6 92.1) (end 87.9 92.1) (width 0.25) (layer F.Cu) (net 4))
 (segment (start 88.81501 92.31501) (end 88.6 92.1) (width 0.25) (layer F.Cu) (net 4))
 (segment (start 87.9 92.1) (end 87.2 92.8) (width 0.25) (layer B.Cu) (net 4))
 (segment (start 87.2 92.8) (end 87.7 93.3) (width 0.25) (layer B.Cu) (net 4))
 (segment (start 86.67 92.27) (end 87.2 92.8) (width 0.25) (layer B.Cu) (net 4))
 (segment (start 92 87.51) (end 92 88.9) (width 0.25) (layer B.Cu) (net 5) (status 400000))
 (segment (start 96.73 89.73) (end 98.35 89.73) (width 0.25) (layer B.Cu) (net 5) (status 800000))
 (segment (start 96.5 89.5) (end 96.73 89.73) (width 0.25) (layer B.Cu) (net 5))
 (segment (start 92.6 89.5) (end 96.5 89.5) (width 0.25) (layer B.Cu) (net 5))
 (segment (start 92 88.9) (end 92.6 89.5) (width 0.25) (layer B.Cu) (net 5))
 (segment (start 85.65 89.73) (end 87.87 89.73) (width 0.25) (layer B.Cu) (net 5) (status 400000))
 (segment (start 91.4 89.5) (end 92 88.9) (width 0.25) (layer B.Cu) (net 5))
 (segment (start 87.87 89.73) (end 88.1 89.5) (width 0.25) (layer B.Cu) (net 5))
 (segment (start 91.72501 98.22501) (end 91.72501 96.42501) (width 0.25) (layer F.Cu) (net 5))
 (segment (start 91.75 98.25) (end 91.72501 98.22501) (width 0.25) (layer F.Cu) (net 5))
 (segment (start 91.75 98.264) (end 91.75 98.25) (width 0.25) (layer F.Cu) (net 5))
 (segment (start 91.37499 96.07499) (end 91.37499 90.47499) (width 0.25) (layer F.Cu) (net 5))
 (segment (start 91.72501 96.42501) (end 91.37499 96.07499) (width 0.25) (layer F.Cu) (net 5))
 (segment (start 91.37499 90.47499) (end 90.7 89.8) (width 0.25) (layer F.Cu) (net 5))
 (segment (start 90.7 89.5) (end 91.4 89.5) (width 0.25) (layer B.Cu) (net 5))
 (via (at 90.7 89.5) (size 0.6) (drill 0.3) (layers F.Cu B.Cu) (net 5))
 (segment (start 90.7 89.8) (end 90.7 89.5) (width 0.25) (layer F.Cu) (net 5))
 (segment (start 88.1 89.5) (end 90.7 89.5) (width 0.25) (layer B.Cu) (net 5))
 (segment (start 94.2 100.3) (end 92.2 100.3) (width 0.25) (layer B.Cu) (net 10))
 (via (at 92.2 100.3) (size 0.6) (drill 0.3) (layers F.Cu B.Cu) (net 10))
 (segment (start 92.325002 100.3) (end 92.925002 99.7) (width 0.25) (layer F.Cu) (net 10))
 (segment (start 92.2 100.3) (end 92.325002 100.3) (width 0.25) (layer F.Cu) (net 10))
 (segment (start 93.27499 98.28899) (end 93.25 98.264) (width 0.25) (layer F.Cu) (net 10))
 (segment (start 93.27499 98.92501) (end 93.27499 98.28899) (width 0.25) (layer F.Cu) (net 10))
 (segment (start 92.925002 99.274998) (end 93.27499 98.92501) (width 0.25) (layer F.Cu) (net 10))
 (segment (start 92.925002 99.7) (end 92.925002 99.274998) (width 0.25) (layer F.Cu) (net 10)))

